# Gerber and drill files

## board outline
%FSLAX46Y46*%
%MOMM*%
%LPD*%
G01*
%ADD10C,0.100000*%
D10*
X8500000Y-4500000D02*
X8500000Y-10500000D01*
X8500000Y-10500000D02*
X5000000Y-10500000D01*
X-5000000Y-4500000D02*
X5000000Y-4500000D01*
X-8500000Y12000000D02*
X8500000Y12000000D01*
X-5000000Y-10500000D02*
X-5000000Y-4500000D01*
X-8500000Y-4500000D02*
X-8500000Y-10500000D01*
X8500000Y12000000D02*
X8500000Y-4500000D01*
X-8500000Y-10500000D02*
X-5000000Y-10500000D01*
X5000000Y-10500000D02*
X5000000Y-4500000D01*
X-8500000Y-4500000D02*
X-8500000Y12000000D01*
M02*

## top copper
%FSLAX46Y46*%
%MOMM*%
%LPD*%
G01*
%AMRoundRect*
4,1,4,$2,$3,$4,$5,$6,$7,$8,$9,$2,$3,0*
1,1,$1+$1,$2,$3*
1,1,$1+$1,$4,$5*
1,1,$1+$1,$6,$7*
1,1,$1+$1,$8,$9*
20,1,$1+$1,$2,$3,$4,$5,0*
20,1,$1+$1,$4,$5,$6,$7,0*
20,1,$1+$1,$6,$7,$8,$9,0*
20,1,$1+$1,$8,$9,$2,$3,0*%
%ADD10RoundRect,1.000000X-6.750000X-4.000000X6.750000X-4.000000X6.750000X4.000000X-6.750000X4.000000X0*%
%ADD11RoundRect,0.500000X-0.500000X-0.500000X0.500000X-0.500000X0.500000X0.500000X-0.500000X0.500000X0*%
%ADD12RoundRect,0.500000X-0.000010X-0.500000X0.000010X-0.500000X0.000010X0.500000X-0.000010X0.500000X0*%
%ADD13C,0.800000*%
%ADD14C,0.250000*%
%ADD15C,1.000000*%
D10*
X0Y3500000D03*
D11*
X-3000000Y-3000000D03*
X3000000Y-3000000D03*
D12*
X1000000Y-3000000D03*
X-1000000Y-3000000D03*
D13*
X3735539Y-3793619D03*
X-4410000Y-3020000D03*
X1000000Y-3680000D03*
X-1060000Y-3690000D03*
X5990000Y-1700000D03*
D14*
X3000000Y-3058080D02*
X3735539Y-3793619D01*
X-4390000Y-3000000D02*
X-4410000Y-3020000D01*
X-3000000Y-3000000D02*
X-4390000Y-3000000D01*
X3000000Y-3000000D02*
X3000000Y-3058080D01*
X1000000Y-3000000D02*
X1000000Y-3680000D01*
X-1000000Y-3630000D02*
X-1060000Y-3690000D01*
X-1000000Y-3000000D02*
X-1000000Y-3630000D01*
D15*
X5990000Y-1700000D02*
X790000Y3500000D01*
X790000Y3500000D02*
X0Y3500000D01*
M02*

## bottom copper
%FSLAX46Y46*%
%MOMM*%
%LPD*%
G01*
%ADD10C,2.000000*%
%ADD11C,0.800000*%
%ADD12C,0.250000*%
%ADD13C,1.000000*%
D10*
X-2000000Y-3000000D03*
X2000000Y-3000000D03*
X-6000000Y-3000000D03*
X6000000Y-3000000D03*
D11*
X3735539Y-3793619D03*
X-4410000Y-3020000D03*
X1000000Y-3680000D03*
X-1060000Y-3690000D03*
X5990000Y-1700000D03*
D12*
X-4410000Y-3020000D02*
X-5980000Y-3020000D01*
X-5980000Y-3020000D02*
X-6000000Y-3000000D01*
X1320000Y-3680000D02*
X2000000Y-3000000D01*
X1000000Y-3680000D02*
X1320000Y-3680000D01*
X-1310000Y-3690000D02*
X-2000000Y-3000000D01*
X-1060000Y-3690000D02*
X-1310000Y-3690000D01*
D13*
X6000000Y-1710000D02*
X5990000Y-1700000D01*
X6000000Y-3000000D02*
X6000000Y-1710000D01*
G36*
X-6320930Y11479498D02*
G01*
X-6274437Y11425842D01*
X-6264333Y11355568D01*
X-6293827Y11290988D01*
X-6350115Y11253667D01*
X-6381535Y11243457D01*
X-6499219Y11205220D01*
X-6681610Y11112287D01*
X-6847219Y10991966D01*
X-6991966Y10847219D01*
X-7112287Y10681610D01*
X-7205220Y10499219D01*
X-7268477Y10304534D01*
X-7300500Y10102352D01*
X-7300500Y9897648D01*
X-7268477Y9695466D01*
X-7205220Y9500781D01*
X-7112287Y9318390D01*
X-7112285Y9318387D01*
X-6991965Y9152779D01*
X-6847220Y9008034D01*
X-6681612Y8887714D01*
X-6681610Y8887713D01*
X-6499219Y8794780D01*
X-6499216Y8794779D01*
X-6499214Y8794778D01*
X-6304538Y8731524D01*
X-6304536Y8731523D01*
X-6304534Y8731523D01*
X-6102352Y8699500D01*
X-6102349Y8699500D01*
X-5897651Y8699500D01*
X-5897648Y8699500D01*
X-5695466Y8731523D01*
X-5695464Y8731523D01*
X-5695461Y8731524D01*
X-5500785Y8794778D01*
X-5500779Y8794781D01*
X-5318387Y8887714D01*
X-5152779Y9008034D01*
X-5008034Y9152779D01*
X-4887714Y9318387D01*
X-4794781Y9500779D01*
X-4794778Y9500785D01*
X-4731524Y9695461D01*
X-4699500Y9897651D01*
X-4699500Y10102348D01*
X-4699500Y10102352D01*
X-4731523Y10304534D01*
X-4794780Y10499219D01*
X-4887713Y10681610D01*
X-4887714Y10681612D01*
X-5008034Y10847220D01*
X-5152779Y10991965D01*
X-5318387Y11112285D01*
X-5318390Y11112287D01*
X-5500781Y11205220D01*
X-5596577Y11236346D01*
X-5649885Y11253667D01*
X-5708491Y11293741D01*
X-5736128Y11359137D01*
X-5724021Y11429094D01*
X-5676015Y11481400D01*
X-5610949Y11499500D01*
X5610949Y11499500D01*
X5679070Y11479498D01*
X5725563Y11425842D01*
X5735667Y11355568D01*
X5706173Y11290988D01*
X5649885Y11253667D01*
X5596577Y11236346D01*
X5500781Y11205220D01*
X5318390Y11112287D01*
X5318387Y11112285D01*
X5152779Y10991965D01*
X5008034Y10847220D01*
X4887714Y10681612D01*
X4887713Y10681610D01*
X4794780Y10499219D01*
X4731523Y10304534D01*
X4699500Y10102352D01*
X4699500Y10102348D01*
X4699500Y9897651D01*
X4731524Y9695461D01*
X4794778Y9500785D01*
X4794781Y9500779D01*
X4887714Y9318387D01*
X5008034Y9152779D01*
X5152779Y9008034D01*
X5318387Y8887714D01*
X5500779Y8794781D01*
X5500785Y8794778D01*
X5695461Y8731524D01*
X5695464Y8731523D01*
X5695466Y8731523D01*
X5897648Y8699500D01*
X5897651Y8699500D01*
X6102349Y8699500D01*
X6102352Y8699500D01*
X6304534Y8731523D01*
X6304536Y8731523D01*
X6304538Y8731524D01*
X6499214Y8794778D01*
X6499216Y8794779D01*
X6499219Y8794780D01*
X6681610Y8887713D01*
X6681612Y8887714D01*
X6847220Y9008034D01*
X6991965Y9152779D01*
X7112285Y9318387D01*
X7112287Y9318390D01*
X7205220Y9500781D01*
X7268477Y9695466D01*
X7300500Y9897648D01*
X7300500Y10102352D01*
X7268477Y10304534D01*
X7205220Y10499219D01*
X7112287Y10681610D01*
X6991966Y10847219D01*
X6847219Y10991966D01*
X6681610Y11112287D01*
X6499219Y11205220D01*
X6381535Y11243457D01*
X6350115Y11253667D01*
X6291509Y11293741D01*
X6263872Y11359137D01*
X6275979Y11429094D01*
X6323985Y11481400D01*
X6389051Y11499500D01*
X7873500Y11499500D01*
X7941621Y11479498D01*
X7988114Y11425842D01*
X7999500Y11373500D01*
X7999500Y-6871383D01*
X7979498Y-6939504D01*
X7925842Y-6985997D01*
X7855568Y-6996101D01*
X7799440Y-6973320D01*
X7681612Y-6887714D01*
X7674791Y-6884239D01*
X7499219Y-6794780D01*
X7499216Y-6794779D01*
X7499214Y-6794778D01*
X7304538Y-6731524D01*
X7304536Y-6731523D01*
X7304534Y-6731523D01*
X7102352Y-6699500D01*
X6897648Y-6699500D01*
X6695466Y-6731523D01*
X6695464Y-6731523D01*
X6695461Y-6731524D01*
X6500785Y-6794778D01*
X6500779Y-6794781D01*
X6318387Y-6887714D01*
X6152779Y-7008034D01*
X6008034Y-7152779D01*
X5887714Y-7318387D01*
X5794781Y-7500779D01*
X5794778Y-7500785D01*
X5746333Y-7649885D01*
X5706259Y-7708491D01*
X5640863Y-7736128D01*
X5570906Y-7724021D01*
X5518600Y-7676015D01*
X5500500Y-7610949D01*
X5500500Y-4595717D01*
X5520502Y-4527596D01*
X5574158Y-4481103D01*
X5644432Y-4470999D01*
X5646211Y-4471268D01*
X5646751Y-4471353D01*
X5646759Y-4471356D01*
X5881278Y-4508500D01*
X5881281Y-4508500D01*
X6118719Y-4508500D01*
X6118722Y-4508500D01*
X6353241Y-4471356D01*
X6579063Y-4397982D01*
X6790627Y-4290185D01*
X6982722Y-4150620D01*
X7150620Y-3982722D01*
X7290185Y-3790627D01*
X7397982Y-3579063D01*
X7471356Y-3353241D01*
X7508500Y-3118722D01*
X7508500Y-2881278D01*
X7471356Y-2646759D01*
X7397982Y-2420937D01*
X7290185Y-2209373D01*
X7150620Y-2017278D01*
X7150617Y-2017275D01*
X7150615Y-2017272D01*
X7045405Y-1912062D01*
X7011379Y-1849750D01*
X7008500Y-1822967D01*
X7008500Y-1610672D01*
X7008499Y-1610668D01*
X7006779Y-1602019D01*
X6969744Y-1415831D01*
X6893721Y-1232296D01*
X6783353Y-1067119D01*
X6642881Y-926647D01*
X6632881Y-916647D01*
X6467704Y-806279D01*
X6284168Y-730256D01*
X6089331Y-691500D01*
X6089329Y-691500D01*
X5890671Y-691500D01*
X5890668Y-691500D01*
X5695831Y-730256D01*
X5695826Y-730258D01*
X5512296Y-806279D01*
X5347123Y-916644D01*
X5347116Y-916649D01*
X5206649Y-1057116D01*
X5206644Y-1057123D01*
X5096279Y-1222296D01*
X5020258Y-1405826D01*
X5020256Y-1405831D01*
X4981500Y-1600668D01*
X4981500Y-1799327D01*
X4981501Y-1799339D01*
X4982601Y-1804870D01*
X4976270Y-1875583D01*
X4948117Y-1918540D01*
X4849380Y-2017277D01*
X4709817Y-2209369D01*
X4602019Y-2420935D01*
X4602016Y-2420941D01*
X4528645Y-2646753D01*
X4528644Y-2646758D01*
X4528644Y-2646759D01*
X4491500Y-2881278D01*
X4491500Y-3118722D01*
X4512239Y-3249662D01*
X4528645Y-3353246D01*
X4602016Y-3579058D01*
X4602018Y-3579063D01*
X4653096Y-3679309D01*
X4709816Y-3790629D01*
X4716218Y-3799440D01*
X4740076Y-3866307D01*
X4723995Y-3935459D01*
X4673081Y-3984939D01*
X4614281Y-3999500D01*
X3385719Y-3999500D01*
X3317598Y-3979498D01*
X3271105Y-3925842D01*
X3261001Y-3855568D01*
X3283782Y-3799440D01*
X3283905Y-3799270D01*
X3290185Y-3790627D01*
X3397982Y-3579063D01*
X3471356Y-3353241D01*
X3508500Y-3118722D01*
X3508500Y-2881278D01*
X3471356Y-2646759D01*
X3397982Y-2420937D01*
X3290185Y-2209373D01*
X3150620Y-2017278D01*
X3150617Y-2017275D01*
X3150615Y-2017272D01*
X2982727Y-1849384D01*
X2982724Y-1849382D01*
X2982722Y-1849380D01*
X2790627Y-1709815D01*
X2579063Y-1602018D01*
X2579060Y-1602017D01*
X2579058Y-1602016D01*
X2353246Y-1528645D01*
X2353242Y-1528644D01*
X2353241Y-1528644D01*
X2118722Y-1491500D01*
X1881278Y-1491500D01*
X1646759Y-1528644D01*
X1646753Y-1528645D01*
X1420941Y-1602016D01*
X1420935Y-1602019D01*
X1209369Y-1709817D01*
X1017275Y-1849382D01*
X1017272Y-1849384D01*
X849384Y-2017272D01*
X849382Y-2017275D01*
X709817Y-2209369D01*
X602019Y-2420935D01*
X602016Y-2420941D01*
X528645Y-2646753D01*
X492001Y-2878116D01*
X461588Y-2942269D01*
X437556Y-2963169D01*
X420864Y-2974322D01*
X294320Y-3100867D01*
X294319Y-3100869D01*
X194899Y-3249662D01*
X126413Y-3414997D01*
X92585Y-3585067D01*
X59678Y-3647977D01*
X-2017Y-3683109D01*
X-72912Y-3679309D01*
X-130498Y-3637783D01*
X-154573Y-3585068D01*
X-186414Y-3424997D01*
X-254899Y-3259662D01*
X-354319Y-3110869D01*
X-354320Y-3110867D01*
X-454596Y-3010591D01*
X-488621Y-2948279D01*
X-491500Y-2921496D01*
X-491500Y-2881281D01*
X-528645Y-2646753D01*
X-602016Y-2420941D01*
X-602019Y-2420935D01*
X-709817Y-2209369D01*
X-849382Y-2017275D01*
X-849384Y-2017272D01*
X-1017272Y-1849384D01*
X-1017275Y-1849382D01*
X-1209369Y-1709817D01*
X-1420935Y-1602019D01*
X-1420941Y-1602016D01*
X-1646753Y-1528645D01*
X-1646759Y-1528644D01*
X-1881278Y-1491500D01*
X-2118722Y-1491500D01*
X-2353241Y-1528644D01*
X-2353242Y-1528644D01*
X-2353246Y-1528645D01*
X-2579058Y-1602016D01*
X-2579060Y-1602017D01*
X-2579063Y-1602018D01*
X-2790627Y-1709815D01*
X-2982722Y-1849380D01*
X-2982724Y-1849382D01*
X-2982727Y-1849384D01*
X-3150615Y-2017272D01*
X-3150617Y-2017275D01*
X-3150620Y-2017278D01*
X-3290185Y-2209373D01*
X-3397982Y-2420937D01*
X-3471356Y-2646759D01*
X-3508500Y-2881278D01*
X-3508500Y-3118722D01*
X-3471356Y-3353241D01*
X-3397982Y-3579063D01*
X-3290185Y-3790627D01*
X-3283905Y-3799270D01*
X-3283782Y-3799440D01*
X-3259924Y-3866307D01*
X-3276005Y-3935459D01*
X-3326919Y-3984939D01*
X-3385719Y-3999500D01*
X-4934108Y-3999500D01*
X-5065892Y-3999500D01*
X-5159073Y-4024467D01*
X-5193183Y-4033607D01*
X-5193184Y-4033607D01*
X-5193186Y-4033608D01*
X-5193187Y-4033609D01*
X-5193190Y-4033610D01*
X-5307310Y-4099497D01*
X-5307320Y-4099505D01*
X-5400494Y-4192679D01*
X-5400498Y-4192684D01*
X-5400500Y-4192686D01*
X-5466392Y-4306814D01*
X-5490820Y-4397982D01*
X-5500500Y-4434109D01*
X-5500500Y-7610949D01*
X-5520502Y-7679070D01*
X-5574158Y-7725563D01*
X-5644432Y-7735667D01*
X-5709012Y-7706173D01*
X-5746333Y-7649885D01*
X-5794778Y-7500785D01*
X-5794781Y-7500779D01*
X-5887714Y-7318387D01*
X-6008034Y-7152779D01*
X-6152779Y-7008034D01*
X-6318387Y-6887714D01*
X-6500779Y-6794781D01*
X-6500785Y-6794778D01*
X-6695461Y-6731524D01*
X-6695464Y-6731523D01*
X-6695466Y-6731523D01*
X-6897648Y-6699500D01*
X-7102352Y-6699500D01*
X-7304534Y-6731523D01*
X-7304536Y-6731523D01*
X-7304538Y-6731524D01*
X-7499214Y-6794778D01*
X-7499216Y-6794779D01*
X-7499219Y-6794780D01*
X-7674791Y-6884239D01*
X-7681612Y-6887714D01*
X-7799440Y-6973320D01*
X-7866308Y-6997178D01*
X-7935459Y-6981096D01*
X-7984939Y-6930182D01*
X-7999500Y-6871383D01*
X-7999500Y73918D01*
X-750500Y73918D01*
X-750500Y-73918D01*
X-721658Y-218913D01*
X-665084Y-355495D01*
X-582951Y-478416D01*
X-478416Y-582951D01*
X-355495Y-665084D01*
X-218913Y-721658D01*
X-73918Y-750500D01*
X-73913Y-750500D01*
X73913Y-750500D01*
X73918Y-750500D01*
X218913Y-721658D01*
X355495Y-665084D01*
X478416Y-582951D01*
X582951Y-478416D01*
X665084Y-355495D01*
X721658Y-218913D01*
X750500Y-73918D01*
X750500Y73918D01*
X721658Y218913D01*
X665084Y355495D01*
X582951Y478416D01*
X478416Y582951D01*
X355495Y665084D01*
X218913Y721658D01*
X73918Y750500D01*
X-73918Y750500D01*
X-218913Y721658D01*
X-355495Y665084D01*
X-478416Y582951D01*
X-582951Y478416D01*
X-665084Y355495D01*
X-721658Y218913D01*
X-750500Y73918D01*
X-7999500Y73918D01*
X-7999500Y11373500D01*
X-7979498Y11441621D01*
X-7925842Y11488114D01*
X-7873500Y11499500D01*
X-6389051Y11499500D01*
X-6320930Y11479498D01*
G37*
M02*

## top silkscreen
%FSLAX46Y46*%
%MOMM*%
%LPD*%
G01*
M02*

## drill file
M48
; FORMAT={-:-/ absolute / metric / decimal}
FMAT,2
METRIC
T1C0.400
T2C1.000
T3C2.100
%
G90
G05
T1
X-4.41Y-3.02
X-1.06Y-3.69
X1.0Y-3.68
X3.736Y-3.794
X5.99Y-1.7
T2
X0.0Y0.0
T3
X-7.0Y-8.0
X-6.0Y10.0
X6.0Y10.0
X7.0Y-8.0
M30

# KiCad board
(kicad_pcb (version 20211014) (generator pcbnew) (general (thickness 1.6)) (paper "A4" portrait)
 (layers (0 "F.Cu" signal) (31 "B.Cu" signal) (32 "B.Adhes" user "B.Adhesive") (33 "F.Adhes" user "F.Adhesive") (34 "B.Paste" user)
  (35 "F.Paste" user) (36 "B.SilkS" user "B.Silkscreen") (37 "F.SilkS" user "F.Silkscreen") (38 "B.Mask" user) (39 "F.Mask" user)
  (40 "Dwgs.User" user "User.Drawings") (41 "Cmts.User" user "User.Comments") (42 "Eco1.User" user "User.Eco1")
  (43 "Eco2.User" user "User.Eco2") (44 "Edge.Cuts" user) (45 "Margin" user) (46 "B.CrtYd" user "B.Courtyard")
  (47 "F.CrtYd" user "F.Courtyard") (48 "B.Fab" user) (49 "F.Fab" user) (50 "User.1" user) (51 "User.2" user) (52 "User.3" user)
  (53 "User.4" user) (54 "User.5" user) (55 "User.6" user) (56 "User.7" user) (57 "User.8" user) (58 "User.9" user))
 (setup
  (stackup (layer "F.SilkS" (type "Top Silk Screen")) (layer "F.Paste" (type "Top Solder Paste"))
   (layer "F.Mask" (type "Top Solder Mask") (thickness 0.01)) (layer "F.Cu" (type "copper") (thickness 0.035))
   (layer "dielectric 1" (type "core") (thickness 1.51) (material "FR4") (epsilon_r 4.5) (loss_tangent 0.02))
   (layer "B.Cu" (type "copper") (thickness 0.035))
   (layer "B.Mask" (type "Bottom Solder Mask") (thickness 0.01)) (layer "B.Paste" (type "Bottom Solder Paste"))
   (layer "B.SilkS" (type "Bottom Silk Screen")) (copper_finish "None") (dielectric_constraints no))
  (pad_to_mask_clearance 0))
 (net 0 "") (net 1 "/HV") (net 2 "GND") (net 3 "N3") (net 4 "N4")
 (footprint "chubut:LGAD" (layer "F.Cu") (at 0 0)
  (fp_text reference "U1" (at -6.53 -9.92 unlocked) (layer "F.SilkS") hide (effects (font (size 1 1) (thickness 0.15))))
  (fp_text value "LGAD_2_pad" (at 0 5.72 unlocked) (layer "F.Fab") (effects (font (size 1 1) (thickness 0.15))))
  (pad "" np_thru_hole circle (at 0 0 90) (size 1 1) (drill 1) (layers F&B.Cu))
  (pad "1" smd roundrect (at 0 -3.5) (size 15.5 10) (layers "F.Cu" "F.Mask") (roundrect_rratio 0.1) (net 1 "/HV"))
  (pad "2" smd roundrect (at -3 3) (size 2 2) (layers "F.Cu" "F.Mask") (roundrect_rratio 0.25) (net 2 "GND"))
  (pad "2" smd roundrect (at 3 3) (size 2 2) (layers "F.Cu" "F.Mask") (roundrect_rratio 0.25) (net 2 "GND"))
  (pad "3" smd roundrect (at 1 3) (size 1 2) (layers "F.Cu" "F.Mask") (roundrect_rratio 0.5) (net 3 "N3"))
  (pad "4" smd roundrect (at -1 3) (size 1 2) (layers "F.Cu" "F.Mask") (roundrect_rratio 0.5) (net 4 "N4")))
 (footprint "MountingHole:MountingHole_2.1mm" (layer "F.Cu") (at -6 -10)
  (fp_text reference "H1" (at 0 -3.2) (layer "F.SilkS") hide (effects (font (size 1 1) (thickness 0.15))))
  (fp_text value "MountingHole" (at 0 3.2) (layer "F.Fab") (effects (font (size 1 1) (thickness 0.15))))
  (pad "" np_thru_hole circle (at 0 0) (size 2.1 2.1) (drill 2.1) (layers *.Cu *.Mask)))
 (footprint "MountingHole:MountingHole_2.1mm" (layer "F.Cu") (at 7 8)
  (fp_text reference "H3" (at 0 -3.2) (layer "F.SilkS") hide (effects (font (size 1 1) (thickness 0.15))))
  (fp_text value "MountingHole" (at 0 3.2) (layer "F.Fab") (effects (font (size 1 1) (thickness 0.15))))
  (pad "" np_thru_hole circle (at 0 0) (size 2.1 2.1) (drill 2.1) (layers *.Cu *.Mask)))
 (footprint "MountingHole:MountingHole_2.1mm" (layer "F.Cu") (at -7 8)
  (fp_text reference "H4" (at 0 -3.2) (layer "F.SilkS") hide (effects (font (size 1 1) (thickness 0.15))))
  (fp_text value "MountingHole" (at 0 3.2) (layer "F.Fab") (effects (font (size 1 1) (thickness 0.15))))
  (pad "" np_thru_hole circle (at 0 0) (size 2.1 2.1) (drill 2.1) (layers *.Cu *.Mask)))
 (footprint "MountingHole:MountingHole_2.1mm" (layer "F.Cu") (at 6 -10)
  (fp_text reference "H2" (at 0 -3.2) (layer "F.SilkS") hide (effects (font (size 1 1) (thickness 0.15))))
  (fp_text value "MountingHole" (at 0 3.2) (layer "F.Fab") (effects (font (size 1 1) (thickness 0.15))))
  (pad "" np_thru_hole circle (at 0 0) (size 2.1 2.1) (drill 2.1) (layers *.Cu *.Mask)))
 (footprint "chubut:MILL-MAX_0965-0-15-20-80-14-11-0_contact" (layer "B.Cu") (at -2 3 180)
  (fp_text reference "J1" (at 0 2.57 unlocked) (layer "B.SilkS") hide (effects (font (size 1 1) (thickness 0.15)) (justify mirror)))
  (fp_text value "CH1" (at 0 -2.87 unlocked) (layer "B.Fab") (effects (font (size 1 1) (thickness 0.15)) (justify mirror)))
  (pad "1" smd circle (at 0 0 180) (size 2 2) (layers "B.Cu" "B.Mask") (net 4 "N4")))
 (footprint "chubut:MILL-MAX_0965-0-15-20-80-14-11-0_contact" (layer "B.Cu") (at 2 3 180)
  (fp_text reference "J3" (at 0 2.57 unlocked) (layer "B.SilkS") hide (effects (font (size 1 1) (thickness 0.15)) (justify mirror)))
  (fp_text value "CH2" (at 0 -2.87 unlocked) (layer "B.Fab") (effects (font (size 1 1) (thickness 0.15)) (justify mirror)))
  (pad "1" smd circle (at 0 0 180) (size 2 2) (layers "B.Cu" "B.Mask") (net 3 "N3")))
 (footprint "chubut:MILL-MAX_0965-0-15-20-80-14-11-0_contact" (layer "B.Cu") (at -6 3 180) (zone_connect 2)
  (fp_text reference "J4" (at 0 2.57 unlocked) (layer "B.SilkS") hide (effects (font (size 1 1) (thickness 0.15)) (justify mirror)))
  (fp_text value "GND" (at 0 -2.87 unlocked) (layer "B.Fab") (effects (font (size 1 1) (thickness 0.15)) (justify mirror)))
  (pad "1" smd circle (at 0 0 180) (size 2 2) (layers "B.Cu" "B.Mask") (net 2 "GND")))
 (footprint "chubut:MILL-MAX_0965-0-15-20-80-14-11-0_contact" (layer "B.Cu") (at 6 3 180)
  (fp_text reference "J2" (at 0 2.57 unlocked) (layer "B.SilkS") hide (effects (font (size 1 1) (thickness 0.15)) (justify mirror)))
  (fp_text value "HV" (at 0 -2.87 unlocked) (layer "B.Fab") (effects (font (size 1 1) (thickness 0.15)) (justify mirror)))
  (pad "1" smd circle (at 0 0 180) (size 2 2) (layers "B.Cu" "B.Mask") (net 1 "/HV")))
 (gr_line (start 8.5 4.5) (end 8.5 10.5) (layer "Edge.Cuts") (width 0.1))
 (gr_line (start 8.5 10.5) (end 5 10.5) (layer "Edge.Cuts") (width 0.1))
 (gr_line (start -5 4.5) (end 5 4.5) (layer "Edge.Cuts") (width 0.1))
 (gr_line (start -8.5 -12) (end 8.5 -12) (layer "Edge.Cuts") (width 0.1))
 (gr_line (start -5 10.5) (end -5 4.5) (layer "Edge.Cuts") (width 0.1))
 (gr_line (start -8.5 4.5) (end -8.5 10.5) (layer "Edge.Cuts") (width 0.1))
 (gr_line (start 8.5 -12) (end 8.5 4.5) (layer "Edge.Cuts") (width 0.1))
 (gr_line (start -8.5 10.5) (end -5 10.5) (layer "Edge.Cuts") (width 0.1))
 (gr_line (start 5 10.5) (end 5 4.5) (layer "Edge.Cuts") (width 0.1))
 (gr_line (start -8.5 4.5) (end -8.5 -12) (layer "Edge.Cuts") (width 0.1))
 (segment (start 3 3.05808) (end 3.735539 3.793619) (width 0.25) (layer "F.Cu") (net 2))
 (segment (start -4.39 3) (end -4.41 3.02) (width 0.25) (layer "F.Cu") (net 2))
 (segment (start -3 3) (end -4.39 3) (width 0.25) (layer "F.Cu") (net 2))
 (segment (start 3 3) (end 3 3.05808) (width 0.25) (layer "F.Cu") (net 2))
 (via (at 3.735539 3.793619) (size 0.8) (drill 0.4) (layers "F.Cu" "B.Cu") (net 2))
 (via (at -4.41 3.02) (size 0.8) (drill 0.4) (layers "F.Cu" "B.Cu") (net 2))
 (segment (start -4.41 3.02) (end -5.98 3.02) (width 0.25) (layer "B.Cu") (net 2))
 (segment (start -5.98 3.02) (end -6 3) (width 0.25) (layer "B.Cu") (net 2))
 (segment (start 1 3) (end 1 3.68) (width 0.25) (layer "F.Cu") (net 3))
 (via (at 1 3.68) (size 0.8) (drill 0.4) (layers "F.Cu" "B.Cu") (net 3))
 (segment (start 1.32 3.68) (end 2 3) (width 0.25) (layer "B.Cu") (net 3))
 (segment (start 1 3.68) (end 1.32 3.68) (width 0.25) (layer "B.Cu") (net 3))
 (segment (start -1 3.63) (end -1.06 3.69) (width 0.25) (layer "F.Cu") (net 4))
 (segment (start -1 3) (end -1 3.63) (width 0.25) (layer "F.Cu") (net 4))
 (via (at -1.06 3.69) (size 0.8) (drill 0.4) (layers "F.Cu" "B.Cu") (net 4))
 (segment (start -1.31 3.69) (end -2 3) (width 0.25) (layer "B.Cu") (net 4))
 (segment (start -1.06 3.69) (end -1.31 3.69) (width 0.25) (layer "B.Cu") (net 4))
 (segment (start 5.99 1.7) (end 0.79 -3.5) (width 1) (layer "F.Cu") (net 1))
 (segment (start 0.79 -3.5) (end 0 -3.5) (width 1) (layer "F.Cu") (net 1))
 (via (at 5.99 1.7) (size 0.8) (drill 0.4) (layers "F.Cu" "B.Cu") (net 1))
 (segment (start 6 1.71) (end 5.99 1.7) (width 1) (layer "B.Cu") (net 1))
 (segment (start 6 3) (end 6 1.71) (width 1) (layer "B.Cu") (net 1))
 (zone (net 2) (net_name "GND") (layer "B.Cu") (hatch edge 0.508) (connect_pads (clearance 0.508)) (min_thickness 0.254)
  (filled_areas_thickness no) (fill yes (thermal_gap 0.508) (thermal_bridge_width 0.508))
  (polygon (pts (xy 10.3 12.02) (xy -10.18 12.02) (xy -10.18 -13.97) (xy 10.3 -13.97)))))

